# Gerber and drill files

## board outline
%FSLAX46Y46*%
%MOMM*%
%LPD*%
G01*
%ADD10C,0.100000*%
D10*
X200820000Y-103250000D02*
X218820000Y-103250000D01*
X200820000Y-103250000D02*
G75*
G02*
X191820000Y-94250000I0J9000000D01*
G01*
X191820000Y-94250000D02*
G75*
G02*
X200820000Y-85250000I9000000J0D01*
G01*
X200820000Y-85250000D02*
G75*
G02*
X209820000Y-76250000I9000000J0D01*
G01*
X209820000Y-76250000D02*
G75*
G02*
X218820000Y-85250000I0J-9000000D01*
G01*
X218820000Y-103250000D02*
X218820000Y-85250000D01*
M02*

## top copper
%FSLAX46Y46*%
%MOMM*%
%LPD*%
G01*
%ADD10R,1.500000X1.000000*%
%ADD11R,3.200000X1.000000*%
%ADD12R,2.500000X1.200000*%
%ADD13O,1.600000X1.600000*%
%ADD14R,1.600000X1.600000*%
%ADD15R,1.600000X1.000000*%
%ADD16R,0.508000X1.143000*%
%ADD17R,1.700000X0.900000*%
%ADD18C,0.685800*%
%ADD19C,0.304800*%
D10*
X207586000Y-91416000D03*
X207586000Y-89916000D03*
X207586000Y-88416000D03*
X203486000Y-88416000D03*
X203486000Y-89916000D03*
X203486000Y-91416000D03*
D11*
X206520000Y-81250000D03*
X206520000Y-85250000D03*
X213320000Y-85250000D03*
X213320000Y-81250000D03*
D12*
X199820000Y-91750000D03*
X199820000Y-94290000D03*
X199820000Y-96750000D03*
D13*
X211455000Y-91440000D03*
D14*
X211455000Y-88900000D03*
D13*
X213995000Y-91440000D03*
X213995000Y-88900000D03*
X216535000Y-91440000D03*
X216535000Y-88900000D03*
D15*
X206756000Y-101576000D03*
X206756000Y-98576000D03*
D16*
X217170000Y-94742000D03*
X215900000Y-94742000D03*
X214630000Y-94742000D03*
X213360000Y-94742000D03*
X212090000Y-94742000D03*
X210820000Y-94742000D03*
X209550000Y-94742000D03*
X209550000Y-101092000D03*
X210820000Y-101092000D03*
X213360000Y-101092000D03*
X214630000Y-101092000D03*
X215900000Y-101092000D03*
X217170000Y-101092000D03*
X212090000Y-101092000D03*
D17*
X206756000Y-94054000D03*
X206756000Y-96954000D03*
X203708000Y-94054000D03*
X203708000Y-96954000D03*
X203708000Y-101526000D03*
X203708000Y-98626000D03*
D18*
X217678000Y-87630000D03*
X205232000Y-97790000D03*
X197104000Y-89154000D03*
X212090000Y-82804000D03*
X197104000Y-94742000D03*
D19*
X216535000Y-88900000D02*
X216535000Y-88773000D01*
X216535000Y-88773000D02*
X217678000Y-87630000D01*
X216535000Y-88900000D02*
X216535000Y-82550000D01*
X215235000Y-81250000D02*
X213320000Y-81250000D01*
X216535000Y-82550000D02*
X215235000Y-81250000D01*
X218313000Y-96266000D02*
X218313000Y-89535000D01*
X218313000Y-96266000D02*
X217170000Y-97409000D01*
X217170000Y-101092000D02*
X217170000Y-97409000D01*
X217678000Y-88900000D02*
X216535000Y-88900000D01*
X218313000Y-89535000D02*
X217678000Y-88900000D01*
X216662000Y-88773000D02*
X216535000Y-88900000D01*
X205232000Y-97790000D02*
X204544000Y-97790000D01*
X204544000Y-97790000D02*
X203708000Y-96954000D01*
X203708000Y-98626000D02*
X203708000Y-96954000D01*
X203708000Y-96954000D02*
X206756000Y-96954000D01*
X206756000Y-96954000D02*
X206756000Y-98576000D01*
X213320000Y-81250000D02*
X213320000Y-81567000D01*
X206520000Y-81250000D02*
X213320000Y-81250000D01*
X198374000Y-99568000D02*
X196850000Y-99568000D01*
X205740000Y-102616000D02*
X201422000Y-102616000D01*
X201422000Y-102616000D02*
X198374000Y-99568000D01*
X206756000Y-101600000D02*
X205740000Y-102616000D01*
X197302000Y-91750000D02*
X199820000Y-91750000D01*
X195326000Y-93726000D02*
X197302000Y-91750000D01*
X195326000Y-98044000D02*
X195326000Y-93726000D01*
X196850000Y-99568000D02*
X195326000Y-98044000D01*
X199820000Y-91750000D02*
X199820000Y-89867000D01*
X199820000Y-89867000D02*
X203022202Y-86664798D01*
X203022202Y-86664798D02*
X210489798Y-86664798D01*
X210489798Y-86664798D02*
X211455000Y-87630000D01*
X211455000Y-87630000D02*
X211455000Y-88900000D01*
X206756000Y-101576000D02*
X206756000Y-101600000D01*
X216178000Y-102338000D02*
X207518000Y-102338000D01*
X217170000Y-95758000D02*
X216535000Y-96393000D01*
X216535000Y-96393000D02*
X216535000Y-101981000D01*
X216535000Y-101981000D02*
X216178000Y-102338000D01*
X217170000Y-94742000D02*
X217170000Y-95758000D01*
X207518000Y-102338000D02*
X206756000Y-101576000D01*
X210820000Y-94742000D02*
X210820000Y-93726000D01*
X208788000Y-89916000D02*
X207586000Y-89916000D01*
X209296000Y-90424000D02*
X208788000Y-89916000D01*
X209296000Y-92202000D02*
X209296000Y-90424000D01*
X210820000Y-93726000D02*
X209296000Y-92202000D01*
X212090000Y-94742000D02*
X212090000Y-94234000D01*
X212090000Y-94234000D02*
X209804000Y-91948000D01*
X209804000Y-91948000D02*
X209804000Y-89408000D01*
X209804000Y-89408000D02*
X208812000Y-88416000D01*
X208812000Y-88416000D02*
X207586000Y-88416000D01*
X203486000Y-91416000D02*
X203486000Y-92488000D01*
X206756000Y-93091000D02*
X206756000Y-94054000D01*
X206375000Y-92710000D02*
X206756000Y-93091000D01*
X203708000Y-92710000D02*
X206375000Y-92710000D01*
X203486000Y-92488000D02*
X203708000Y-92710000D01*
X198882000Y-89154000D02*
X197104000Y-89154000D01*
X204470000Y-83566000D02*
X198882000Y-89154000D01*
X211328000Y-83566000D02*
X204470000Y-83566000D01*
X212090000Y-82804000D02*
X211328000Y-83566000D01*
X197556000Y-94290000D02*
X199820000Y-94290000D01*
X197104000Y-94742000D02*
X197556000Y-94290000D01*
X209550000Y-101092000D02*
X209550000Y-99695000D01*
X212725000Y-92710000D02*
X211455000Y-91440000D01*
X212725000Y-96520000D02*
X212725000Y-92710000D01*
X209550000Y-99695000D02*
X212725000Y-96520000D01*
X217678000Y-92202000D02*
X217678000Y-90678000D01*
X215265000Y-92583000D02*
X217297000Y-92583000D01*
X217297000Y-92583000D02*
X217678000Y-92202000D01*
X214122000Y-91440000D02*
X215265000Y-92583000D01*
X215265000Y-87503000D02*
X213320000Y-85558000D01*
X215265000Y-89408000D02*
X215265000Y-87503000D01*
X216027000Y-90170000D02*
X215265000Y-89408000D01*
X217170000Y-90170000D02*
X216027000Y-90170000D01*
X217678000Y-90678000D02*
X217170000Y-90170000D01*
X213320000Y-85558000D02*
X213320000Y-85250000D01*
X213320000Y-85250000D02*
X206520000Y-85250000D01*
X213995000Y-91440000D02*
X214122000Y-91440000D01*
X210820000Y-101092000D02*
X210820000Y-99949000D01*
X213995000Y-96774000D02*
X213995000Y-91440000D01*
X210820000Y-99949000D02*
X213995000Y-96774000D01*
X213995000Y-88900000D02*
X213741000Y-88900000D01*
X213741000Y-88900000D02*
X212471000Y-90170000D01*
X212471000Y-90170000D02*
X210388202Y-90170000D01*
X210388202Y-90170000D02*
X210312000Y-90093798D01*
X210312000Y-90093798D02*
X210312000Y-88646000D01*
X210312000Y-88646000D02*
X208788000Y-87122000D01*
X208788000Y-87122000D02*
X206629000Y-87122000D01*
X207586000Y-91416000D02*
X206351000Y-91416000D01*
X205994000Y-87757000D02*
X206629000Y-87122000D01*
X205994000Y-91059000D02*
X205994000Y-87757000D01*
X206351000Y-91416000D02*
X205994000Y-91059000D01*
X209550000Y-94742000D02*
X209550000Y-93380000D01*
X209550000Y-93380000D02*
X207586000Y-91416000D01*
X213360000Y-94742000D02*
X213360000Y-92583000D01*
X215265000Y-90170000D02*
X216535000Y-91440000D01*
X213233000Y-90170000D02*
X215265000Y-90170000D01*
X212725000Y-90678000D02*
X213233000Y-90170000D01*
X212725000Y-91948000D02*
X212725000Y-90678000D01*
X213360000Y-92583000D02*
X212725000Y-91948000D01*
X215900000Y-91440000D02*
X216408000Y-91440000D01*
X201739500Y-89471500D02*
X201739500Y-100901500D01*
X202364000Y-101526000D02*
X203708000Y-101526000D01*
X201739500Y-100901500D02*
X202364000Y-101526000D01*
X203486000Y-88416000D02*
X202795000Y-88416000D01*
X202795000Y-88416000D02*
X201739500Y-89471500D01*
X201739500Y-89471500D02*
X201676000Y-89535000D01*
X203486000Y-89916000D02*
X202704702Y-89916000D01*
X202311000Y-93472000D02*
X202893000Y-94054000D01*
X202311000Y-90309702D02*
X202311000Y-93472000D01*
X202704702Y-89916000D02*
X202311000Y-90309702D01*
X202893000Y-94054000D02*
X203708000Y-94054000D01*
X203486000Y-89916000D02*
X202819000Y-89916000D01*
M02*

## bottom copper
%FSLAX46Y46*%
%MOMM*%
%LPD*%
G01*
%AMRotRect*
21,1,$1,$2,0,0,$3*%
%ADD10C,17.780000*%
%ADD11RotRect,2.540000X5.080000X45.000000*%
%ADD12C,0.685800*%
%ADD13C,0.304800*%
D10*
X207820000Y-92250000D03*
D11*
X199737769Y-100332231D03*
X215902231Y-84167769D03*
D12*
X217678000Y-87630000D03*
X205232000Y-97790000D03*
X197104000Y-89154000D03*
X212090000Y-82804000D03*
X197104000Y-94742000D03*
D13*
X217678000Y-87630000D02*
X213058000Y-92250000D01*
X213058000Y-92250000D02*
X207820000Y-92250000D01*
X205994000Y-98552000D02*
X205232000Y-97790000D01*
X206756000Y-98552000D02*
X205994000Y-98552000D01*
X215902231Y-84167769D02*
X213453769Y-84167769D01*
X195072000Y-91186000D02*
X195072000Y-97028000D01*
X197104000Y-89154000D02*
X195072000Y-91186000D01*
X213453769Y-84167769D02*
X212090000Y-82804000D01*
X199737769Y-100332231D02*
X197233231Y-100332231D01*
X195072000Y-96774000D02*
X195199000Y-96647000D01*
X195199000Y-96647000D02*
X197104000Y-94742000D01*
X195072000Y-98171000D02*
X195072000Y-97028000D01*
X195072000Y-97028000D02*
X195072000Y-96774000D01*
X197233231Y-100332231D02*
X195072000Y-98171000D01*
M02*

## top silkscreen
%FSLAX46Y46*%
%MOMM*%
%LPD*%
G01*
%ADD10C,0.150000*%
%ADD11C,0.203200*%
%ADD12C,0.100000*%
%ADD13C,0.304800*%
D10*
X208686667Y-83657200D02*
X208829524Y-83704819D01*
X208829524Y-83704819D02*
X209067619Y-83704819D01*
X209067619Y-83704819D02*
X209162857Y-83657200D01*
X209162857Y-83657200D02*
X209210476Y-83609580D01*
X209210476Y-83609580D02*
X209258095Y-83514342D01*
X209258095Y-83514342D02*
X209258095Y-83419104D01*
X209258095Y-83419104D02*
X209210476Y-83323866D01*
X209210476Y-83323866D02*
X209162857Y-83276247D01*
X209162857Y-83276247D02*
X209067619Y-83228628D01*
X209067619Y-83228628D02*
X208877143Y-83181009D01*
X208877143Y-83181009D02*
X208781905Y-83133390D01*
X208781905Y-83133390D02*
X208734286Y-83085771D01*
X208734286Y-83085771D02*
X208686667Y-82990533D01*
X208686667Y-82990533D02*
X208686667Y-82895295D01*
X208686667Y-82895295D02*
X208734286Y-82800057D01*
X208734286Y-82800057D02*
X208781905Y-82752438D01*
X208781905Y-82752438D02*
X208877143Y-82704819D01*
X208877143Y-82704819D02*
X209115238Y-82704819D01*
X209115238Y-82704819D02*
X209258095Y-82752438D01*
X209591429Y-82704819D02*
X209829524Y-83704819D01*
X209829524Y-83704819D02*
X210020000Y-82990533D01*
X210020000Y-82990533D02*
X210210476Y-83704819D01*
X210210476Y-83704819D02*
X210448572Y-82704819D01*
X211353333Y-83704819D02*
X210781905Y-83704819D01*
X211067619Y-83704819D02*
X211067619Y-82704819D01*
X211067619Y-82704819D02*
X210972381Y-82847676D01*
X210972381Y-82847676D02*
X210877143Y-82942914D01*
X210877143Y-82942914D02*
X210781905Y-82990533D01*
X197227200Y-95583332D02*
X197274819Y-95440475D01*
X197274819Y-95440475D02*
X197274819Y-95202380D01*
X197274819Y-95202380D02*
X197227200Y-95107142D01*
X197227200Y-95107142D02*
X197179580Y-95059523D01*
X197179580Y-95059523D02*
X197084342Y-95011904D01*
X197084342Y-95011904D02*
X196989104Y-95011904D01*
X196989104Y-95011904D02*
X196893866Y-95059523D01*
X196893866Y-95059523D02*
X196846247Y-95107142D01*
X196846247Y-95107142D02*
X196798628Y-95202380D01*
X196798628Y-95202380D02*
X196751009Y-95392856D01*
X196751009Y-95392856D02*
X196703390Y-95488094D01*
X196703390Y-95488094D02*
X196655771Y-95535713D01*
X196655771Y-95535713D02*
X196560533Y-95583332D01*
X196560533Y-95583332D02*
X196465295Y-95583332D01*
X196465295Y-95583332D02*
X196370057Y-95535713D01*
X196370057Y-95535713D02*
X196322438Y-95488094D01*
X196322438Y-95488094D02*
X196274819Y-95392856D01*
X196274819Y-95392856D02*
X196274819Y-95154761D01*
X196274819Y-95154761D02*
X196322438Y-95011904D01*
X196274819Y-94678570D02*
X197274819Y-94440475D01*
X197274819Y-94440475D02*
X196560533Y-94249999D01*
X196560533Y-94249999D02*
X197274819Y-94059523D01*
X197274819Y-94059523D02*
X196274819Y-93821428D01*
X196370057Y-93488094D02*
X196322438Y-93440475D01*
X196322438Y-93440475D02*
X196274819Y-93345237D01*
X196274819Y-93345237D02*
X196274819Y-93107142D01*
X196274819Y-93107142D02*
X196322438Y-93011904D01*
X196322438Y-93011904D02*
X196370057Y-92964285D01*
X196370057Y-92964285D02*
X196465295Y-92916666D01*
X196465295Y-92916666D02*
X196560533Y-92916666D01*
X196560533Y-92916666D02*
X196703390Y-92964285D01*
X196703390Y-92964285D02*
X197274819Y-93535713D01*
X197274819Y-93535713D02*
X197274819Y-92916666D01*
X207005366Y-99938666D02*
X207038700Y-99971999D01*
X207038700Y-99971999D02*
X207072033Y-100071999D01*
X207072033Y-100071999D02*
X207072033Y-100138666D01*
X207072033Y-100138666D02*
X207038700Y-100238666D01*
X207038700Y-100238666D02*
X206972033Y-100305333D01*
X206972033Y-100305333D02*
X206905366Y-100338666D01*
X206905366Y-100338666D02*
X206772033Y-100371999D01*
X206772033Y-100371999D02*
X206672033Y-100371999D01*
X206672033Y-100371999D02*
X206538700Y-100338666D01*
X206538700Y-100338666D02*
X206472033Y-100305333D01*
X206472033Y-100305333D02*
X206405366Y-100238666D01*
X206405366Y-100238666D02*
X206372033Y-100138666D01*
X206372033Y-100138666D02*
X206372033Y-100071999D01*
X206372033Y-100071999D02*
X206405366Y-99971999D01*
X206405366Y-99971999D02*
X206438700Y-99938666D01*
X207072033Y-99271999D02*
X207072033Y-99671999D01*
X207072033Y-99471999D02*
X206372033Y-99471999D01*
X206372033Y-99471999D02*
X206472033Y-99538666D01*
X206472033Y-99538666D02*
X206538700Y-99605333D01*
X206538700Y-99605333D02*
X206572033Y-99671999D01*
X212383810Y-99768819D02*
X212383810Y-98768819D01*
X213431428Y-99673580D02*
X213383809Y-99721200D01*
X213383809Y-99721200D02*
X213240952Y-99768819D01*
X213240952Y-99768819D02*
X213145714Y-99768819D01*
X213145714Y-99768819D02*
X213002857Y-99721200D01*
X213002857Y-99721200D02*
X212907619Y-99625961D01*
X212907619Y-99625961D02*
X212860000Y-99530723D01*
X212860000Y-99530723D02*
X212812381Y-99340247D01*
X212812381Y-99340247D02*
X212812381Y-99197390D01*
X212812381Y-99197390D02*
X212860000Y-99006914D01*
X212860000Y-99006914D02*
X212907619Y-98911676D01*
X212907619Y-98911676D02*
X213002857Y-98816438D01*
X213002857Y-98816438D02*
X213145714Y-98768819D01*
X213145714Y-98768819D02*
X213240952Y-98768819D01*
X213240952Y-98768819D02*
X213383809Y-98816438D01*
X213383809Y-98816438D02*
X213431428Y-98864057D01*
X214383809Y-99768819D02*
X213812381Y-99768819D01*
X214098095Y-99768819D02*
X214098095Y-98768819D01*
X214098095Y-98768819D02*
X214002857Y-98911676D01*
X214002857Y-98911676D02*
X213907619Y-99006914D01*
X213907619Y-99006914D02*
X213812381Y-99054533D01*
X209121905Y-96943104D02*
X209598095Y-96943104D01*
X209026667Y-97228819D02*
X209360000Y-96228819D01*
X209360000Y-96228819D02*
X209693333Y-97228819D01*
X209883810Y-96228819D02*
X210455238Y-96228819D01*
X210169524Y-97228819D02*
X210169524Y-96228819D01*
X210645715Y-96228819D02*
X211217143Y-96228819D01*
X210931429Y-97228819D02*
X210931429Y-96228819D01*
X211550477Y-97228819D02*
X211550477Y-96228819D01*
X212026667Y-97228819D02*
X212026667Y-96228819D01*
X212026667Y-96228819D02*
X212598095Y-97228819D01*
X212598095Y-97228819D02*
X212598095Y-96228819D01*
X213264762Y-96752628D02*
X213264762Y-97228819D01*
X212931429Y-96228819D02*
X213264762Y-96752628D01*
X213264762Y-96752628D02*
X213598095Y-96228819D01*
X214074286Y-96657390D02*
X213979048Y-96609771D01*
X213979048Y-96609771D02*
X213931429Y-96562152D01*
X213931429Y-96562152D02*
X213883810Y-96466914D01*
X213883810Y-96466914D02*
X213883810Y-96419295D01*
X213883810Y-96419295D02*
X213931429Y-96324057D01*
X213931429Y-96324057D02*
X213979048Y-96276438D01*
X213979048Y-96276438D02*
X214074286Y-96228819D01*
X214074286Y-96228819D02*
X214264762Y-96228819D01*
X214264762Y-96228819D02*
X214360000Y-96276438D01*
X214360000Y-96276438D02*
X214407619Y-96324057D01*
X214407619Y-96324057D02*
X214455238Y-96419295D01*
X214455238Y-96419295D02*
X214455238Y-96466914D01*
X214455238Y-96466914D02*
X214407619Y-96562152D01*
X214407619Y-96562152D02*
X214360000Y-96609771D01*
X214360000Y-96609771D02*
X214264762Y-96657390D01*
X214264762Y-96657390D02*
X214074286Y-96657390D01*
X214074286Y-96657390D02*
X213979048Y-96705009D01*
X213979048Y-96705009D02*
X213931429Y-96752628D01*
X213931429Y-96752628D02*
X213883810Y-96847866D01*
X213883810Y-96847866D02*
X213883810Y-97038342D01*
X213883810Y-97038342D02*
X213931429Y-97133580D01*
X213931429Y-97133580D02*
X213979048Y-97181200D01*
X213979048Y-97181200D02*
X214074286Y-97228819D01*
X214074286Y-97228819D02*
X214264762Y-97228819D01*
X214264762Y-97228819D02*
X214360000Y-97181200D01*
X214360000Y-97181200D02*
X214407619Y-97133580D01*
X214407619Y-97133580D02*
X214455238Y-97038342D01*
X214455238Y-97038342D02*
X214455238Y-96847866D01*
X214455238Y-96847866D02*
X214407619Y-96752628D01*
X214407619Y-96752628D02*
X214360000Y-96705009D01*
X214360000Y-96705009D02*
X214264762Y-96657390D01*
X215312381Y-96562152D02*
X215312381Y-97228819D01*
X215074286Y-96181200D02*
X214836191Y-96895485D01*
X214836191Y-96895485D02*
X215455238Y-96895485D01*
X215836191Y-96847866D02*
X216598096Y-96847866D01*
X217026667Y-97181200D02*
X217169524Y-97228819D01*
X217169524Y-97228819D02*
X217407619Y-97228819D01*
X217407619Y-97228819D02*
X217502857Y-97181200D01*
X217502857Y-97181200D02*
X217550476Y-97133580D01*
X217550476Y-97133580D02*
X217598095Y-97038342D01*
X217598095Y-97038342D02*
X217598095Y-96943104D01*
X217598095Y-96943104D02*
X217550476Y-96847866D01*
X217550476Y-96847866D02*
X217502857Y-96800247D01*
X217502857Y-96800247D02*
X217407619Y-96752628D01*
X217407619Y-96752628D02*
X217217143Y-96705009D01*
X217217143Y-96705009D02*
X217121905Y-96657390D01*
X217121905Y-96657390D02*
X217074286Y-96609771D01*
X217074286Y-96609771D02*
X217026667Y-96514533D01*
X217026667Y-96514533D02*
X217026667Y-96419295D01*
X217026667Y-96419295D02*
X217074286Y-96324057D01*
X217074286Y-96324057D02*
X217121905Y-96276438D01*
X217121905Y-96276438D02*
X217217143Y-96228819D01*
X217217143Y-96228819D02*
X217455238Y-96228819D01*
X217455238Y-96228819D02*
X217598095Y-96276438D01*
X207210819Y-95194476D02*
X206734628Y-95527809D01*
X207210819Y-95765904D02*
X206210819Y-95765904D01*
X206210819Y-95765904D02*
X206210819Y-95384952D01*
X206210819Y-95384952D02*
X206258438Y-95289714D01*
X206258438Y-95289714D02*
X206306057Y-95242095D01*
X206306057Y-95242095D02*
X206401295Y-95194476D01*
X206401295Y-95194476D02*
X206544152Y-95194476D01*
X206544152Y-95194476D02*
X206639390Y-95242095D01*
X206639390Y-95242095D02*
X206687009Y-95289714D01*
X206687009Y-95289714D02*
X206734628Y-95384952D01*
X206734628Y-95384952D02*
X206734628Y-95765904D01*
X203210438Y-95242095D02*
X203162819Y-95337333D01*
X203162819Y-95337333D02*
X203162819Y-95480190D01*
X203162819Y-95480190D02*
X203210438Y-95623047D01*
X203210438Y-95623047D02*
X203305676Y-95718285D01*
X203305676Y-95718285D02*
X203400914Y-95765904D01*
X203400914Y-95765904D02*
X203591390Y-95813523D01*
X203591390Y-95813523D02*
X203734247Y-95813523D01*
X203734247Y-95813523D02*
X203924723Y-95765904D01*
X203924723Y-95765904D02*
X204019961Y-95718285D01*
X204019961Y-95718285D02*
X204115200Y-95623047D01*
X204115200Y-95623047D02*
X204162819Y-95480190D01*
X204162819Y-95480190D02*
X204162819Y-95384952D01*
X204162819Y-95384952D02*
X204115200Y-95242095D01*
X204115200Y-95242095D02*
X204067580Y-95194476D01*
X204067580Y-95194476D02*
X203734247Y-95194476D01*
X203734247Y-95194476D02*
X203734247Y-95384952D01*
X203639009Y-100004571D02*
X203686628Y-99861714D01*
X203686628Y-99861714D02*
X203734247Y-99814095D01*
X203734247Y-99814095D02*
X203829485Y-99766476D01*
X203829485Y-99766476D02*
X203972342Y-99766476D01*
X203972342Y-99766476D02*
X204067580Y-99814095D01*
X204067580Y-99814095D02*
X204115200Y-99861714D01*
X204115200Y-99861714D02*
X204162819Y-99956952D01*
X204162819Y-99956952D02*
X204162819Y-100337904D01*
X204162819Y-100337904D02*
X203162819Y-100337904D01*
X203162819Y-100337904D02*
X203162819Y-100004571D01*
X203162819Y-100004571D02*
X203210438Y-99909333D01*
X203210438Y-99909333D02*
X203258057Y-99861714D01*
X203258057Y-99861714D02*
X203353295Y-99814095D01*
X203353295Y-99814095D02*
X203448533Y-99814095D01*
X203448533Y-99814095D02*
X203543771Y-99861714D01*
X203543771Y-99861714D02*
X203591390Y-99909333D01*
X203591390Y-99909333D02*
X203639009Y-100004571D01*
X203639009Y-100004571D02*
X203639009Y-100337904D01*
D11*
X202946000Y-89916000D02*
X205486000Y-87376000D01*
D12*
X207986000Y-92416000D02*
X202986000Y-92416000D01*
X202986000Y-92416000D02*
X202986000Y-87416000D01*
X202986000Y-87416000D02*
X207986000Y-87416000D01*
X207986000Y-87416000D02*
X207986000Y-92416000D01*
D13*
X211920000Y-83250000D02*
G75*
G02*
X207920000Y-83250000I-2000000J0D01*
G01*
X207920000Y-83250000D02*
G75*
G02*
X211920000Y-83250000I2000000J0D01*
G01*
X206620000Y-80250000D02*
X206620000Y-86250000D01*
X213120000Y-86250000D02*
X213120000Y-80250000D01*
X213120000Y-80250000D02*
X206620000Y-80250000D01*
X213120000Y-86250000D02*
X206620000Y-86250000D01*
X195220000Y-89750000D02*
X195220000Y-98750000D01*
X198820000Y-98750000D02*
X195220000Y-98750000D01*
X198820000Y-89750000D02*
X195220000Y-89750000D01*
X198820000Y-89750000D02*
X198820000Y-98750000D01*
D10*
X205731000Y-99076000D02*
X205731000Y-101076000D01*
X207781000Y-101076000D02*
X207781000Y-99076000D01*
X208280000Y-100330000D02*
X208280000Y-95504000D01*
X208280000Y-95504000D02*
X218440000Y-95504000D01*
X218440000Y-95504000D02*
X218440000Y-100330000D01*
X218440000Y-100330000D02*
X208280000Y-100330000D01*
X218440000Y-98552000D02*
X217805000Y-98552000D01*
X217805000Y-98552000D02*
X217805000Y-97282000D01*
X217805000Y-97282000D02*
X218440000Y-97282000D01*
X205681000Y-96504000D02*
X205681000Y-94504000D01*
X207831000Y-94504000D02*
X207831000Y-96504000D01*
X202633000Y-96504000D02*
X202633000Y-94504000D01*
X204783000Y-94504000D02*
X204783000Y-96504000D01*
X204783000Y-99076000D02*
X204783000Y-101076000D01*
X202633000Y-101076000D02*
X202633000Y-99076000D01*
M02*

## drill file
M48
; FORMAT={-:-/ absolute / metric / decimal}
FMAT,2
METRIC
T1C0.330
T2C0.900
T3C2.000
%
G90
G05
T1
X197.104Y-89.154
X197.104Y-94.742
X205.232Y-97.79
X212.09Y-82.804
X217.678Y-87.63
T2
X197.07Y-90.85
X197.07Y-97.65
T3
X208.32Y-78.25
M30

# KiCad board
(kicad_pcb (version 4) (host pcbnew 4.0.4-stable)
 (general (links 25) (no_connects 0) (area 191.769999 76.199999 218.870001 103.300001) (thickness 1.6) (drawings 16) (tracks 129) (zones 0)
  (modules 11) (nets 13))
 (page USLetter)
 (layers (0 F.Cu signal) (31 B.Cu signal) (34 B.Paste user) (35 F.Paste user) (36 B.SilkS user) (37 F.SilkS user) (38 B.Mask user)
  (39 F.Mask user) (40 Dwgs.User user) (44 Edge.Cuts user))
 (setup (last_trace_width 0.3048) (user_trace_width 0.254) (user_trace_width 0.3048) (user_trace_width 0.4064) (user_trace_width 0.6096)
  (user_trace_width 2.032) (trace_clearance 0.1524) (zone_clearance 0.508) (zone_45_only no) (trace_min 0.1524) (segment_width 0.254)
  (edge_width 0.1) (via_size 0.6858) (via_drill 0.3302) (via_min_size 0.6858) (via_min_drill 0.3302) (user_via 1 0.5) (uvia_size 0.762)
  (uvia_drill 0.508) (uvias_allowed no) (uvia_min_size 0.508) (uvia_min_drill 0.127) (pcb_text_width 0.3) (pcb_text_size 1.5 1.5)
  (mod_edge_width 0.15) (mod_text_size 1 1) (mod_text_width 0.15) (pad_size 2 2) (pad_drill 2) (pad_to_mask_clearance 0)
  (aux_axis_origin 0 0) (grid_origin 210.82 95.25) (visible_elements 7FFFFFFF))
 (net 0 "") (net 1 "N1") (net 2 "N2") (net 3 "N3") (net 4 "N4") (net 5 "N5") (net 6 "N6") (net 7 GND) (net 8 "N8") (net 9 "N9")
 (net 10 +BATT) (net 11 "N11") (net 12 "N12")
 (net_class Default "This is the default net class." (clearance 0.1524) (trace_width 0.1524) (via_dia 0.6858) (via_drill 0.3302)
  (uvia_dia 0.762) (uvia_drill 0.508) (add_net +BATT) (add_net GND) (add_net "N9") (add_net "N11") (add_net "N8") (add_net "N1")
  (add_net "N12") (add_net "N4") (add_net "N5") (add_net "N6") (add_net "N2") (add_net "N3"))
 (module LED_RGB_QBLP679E (layer F.Cu) (at 205.486 89.916 180)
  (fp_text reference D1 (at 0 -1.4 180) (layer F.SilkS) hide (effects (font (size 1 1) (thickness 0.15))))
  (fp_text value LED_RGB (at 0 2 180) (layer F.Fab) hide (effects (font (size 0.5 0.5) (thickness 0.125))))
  (fp_line (start 2.54 0) (end 0 2.54) (layer F.SilkS) (width 0.2032))
  (fp_line (start -2.5 -2.5) (end 2.5 -2.5) (layer F.SilkS) (width 0.1))
  (fp_line (start 2.5 -2.5) (end 2.5 2.5) (layer F.SilkS) (width 0.1))
  (fp_line (start 2.5 2.5) (end -2.5 2.5) (layer F.SilkS) (width 0.1))
  (fp_line (start -2.5 2.5) (end -2.5 -2.5) (layer F.SilkS) (width 0.1))
  (pad 4 smd rect (at -2.1 -1.5 270) (size 1 1.5) (layers F.Cu F.Paste F.Mask) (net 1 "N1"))
  (pad 5 smd rect (at -2.1 0 270) (size 1 1.5) (layers F.Cu F.Paste F.Mask) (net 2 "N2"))
  (pad 6 smd rect (at -2.1 1.5 270) (size 1 1.5) (layers F.Cu F.Paste F.Mask) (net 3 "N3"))
  (pad 1 smd rect (at 2 1.5 270) (size 1 1.5) (layers F.Cu F.Paste F.Mask) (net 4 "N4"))
  (pad 2 smd rect (at 2 0 270) (size 1 1.5) (layers F.Cu F.Paste F.Mask) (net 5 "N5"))
  (pad 3 smd rect (at 2 -1.5 270) (size 1 1.5) (layers F.Cu F.Paste F.Mask) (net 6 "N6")))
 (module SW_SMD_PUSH (layer F.Cu) (at 213.32 85.25 180)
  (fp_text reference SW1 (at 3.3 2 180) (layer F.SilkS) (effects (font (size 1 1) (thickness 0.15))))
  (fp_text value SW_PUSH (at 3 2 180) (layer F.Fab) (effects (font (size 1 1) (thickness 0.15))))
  (fp_circle (center 3.4 2) (end 3.4 0) (layer F.SilkS) (width 0.3048))
  (fp_line (start 6.7 5) (end 6.7 -1) (layer F.SilkS) (width 0.3048))
  (fp_line (start 0.2 -1) (end 0.2 5) (layer F.SilkS) (width 0.3048))
  (fp_line (start 0.2 5) (end 6.7 5) (layer F.SilkS) (width 0.3048))
  (fp_line (start 0.2 -1) (end 6.7 -1) (layer F.SilkS) (width 0.3048))
  (pad 2 smd rect (at 6.8 4 180) (size 3.2 1) (layers F.Cu F.Paste F.Mask) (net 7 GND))
  (pad 1 smd rect (at 6.8 0 180) (size 3.2 1) (layers F.Cu F.Paste F.Mask) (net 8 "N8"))
  (pad 1 smd rect (at 0 0 180) (size 3.2 1) (layers F.Cu F.Paste F.Mask) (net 8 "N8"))
  (pad 2 smd rect (at 0 4 180) (size 3.2 1) (layers F.Cu F.Paste F.Mask) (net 7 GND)))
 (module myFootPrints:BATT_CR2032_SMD (layer B.Cu) (at 207.82 92.25 45)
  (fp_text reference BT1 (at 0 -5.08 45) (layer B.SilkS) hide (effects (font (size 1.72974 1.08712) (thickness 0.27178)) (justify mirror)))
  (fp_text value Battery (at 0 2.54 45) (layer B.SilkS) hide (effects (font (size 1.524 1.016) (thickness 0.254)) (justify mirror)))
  (pad 2 smd circle (at 0 0 45) (size 17.78 17.78) (layers B.Cu B.Paste B.Mask) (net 7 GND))
  (pad 1 smd rect (at -11.43 0 45) (size 2.54 5.08) (layers B.Cu B.Paste B.Mask) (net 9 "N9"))
  (pad 1 smd rect (at 11.43 0 45) (size 2.54 5.08) (layers B.Cu B.Paste B.Mask) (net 9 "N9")))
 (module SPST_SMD (layer F.Cu) (at 199.82 94.25 270)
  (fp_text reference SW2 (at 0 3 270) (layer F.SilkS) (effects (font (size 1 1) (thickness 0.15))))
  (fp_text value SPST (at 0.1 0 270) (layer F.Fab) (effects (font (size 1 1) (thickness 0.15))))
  (fp_line (start -4.5 4.6) (end 4.5 4.6) (layer F.SilkS) (width 0.3048))
  (fp_line (start 4.5 1) (end 4.5 4.6) (layer F.SilkS) (width 0.3048))
  (fp_line (start -4.5 1) (end -4.5 4.6) (layer F.SilkS) (width 0.3048))
  (fp_line (start -4.5 1) (end 4.5 1) (layer F.SilkS) (width 0.3048))
  (pad "" np_thru_hole circle (at 3.4 2.75 270) (size 0.9 0.9) (drill 0.9) (layers *.Cu *.Mask))
  (pad 1 smd rect (at -2.5 0 270) (size 1.2 2.5) (layers F.Cu F.Paste F.Mask) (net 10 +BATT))
  (pad 2 smd rect (at 0.04 0 270) (size 1.2 2.5) (layers F.Cu F.Paste F.Mask) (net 9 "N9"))
  (pad 3 smd rect (at 2.5 0 270) (size 1.2 2.5) (layers F.Cu F.Paste F.Mask))
  (pad "" np_thru_hole circle (at -3.4 2.75 270) (size 0.9 0.9) (drill 0.9) (layers *.Cu *.Mask)))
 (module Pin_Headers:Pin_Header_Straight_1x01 (layer F.Cu) (at 208.32 78.25)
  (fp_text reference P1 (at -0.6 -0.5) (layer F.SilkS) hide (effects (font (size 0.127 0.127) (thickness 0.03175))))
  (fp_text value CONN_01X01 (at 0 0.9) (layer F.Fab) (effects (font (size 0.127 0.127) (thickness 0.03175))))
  (pad "" np_thru_hole circle (at 0 0) (size 2 2) (drill 2) (layers *.Cu *.Mask)))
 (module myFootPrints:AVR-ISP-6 (layer F.Cu) (at 211.455 91.44 90)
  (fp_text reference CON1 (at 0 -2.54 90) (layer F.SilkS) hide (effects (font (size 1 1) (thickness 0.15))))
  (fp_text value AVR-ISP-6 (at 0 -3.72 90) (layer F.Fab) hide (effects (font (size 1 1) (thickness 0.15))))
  (pad 1 smd oval (at 0 0 90) (size 1.6 1.6) (layers F.Cu F.Paste F.Mask) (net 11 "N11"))
  (pad 2 smd rect (at 2.54 0 90) (size 1.6 1.6) (layers F.Cu F.Paste F.Mask) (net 10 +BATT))
  (pad 3 smd oval (at 0 2.54 90) (size 1.6 1.6) (layers F.Cu F.Paste F.Mask) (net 8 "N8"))
  (pad 4 smd oval (at 2.54 2.54 90) (size 1.6 1.6) (layers F.Cu F.Paste F.Mask) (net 1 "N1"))
  (pad 5 smd oval (at 0 5.08 90) (size 1.6 1.6) (layers F.Cu F.Paste F.Mask) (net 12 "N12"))
  (pad 6 smd oval (at 2.54 5.08 90) (size 1.6 1.6) (layers F.Cu F.Paste F.Mask) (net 7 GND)))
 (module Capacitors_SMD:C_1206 (layer F.Cu) (at 206.756 100.076 90)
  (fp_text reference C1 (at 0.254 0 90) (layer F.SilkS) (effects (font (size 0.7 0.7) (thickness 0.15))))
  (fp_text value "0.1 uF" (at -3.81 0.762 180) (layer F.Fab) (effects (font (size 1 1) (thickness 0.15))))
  (fp_line (start 1 -1.025) (end -1 -1.025) (layer F.SilkS) (width 0.15))
  (fp_line (start -1 1.025) (end 1 1.025) (layer F.SilkS) (width 0.15))
  (pad 1 smd rect (at -1.5 0 90) (size 1 1.6) (layers F.Cu F.Paste F.Mask) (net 10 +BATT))
  (pad 2 smd rect (at 1.5 0 90) (size 1 1.6) (layers F.Cu F.Paste F.Mask) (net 7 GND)))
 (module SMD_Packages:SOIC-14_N (layer F.Cu) (at 213.36 98.044 180)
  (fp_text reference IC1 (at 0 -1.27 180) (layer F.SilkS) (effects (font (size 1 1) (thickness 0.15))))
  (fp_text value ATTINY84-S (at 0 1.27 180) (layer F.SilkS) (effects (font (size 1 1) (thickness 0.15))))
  (fp_line (start 5.08 -2.286) (end 5.08 2.54) (layer F.SilkS) (width 0.15))
  (fp_line (start 5.08 2.54) (end -5.08 2.54) (layer F.SilkS) (width 0.15))
  (fp_line (start -5.08 2.54) (end -5.08 -2.286) (layer F.SilkS) (width 0.15))
  (fp_line (start -5.08 -2.286) (end 5.08 -2.286) (layer F.SilkS) (width 0.15))
  (fp_line (start -5.08 -0.508) (end -4.445 -0.508) (layer F.SilkS) (width 0.15))
  (fp_line (start -4.445 -0.508) (end -4.445 0.762) (layer F.SilkS) (width 0.15))
  (fp_line (start -4.445 0.762) (end -5.08 0.762) (layer F.SilkS) (width 0.15))
  (pad 1 smd rect (at -3.81 3.302 180) (size 0.508 1.143) (layers F.Cu F.Paste F.Mask) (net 10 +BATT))
  (pad 2 smd rect (at -2.54 3.302 180) (size 0.508 1.143) (layers F.Cu F.Paste F.Mask))
  (pad 3 smd rect (at -1.27 3.302 180) (size 0.508 1.143) (layers F.Cu F.Paste F.Mask))
  (pad 4 smd rect (at 0 3.302 180) (size 0.508 1.143) (layers F.Cu F.Paste F.Mask) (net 12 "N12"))
  (pad 5 smd rect (at 1.27 3.302 180) (size 0.508 1.143) (layers F.Cu F.Paste F.Mask) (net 3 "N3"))
  (pad 6 smd rect (at 2.54 3.302 180) (size 0.508 1.143) (layers F.Cu F.Paste F.Mask) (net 2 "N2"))
  (pad 7 smd rect (at 3.81 3.302 180) (size 0.508 1.143) (layers F.Cu F.Paste F.Mask) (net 1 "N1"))
  (pad 8 smd rect (at 3.81 -3.048 180) (size 0.508 1.143) (layers F.Cu F.Paste F.Mask) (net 11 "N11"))
  (pad 9 smd rect (at 2.54 -3.048 180) (size 0.508 1.143) (layers F.Cu F.Paste F.Mask) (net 8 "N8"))
  (pad 11 smd rect (at 0 -3.048 180) (size 0.508 1.143) (layers F.Cu F.Paste F.Mask))
  (pad 12 smd rect (at -1.27 -3.048 180) (size 0.508 1.143) (layers F.Cu F.Paste F.Mask))
  (pad 13 smd rect (at -2.54 -3.048 180) (size 0.508 1.143) (layers F.Cu F.Paste F.Mask))
  (pad 14 smd rect (at -3.81 -3.048 180) (size 0.508 1.143) (layers F.Cu F.Paste F.Mask) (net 7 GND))
  (pad 10 smd rect (at 1.27 -3.048 180) (size 0.508 1.143) (layers F.Cu F.Paste F.Mask)))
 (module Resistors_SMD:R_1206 (layer F.Cu) (at 206.756 95.504 270)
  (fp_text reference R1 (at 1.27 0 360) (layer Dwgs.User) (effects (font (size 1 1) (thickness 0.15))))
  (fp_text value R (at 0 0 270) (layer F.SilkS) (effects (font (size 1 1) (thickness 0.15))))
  (fp_line (start 1 1.075) (end -1 1.075) (layer F.SilkS) (width 0.15))
  (fp_line (start -1 -1.075) (end 1 -1.075) (layer F.SilkS) (width 0.15))
  (pad 1 smd rect (at -1.45 0 270) (size 0.9 1.7) (layers F.Cu F.Paste F.Mask) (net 6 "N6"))
  (pad 2 smd rect (at 1.45 0 270) (size 0.9 1.7) (layers F.Cu F.Paste F.Mask) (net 7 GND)))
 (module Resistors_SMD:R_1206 (layer F.Cu) (at 203.708 95.504 270)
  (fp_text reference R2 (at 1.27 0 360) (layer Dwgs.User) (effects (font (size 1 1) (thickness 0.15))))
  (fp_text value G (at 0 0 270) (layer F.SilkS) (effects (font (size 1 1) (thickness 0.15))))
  (fp_line (start 1 1.075) (end -1 1.075) (layer F.SilkS) (width 0.15))
  (fp_line (start -1 -1.075) (end 1 -1.075) (layer F.SilkS) (width 0.15))
  (pad 1 smd rect (at -1.45 0 270) (size 0.9 1.7) (layers F.Cu F.Paste F.Mask) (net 5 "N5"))
  (pad 2 smd rect (at 1.45 0 270) (size 0.9 1.7) (layers F.Cu F.Paste F.Mask) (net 7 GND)))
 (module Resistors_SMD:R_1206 (layer F.Cu) (at 203.708 100.076 90)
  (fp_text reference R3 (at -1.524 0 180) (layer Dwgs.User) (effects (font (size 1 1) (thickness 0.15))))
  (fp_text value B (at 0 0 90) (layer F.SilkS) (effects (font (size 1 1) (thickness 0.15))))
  (fp_line (start 1 1.075) (end -1 1.075) (layer F.SilkS) (width 0.15))
  (fp_line (start -1 -1.075) (end 1 -1.075) (layer F.SilkS) (width 0.15))
  (pad 1 smd rect (at -1.45 0 90) (size 0.9 1.7) (layers F.Cu F.Paste F.Mask) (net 4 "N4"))
  (pad 2 smd rect (at 1.45 0 90) (size 0.9 1.7) (layers F.Cu F.Paste F.Mask) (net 7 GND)))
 (gr_line (start 200.82 103.25) (end 218.82 103.25) (angle 90) (layer Edge.Cuts) (width 0.1))
 (gr_arc (start 200.82 94.25) (end 200.82 103.25) (angle 90) (layer Edge.Cuts) (width 0.1))
 (gr_arc (start 200.82 94.25) (end 191.82 94.25) (angle 90) (layer Edge.Cuts) (width 0.1))
 (gr_arc (start 209.82 85.25) (end 200.82 85.25) (angle 90) (layer Edge.Cuts) (width 0.1))
 (gr_arc (start 209.82 85.25) (end 209.82 76.25) (angle 90) (layer Edge.Cuts) (width 0.1))
 (gr_line (start 218.82 103.25) (end 218.82 85.25) (angle 90) (layer Edge.Cuts) (width 0.1))
 (segment (start 216.535 88.9) (end 216.535 88.773) (width 0.3048) (layer F.Cu) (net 7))
 (segment (start 216.535 88.773) (end 217.678 87.63) (width 0.3048) (layer F.Cu) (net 7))
 (segment (start 217.678 87.63) (end 213.058 92.25) (width 0.3048) (layer B.Cu) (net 7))
 (via (at 217.678 87.63) (size 0.6858) (drill 0.3302) (layers F.Cu B.Cu) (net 7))
 (segment (start 213.058 92.25) (end 207.82 92.25) (width 0.3048) (layer B.Cu) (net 7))
 (segment (start 216.535 88.9) (end 216.535 82.55) (width 0.3048) (layer F.Cu) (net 7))
 (segment (start 215.235 81.25) (end 213.32 81.25) (width 0.3048) (layer F.Cu) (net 7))
 (segment (start 216.535 82.55) (end 215.235 81.25) (width 0.3048) (layer F.Cu) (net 7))
 (segment (start 218.313 96.266) (end 218.313 89.535) (width 0.3048) (layer F.Cu) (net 7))
 (segment (start 218.313 96.266) (end 217.17 97.409) (width 0.3048) (layer F.Cu) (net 7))
 (segment (start 217.17 101.092) (end 217.17 97.409) (width 0.3048) (layer F.Cu) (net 7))
 (segment (start 217.678 88.9) (end 216.535 88.9) (width 0.3048) (layer F.Cu) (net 7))
 (segment (start 218.313 89.535) (end 217.678 88.9) (width 0.3048) (layer F.Cu) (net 7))
 (segment (start 216.662 88.773) (end 216.535 88.9) (width 0.3048) (layer F.Cu) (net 7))
 (segment (start 205.232 97.79) (end 204.544 97.79) (width 0.3048) (layer F.Cu) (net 7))
 (segment (start 205.994 98.552) (end 205.232 97.79) (width 0.3048) (layer B.Cu) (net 7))
 (via (at 205.232 97.79) (size 0.6858) (drill 0.3302) (layers F.Cu B.Cu) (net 7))
 (segment (start 204.544 97.79) (end 203.708 96.954) (width 0.3048) (layer F.Cu) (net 7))
 (segment (start 206.756 98.552) (end 205.994 98.552) (width 0.3048) (layer B.Cu) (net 7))
 (segment (start 203.708 98.626) (end 203.708 96.954) (width 0.3048) (layer F.Cu) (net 7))
 (segment (start 203.708 96.954) (end 206.756 96.954) (width 0.3048) (layer F.Cu) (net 7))
 (segment (start 206.756 96.954) (end 206.756 98.576) (width 0.3048) (layer F.Cu) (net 7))
 (segment (start 213.32 81.25) (end 213.32 81.567) (width 0.3048) (layer F.Cu) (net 7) (status 30))
 (segment (start 206.52 81.25) (end 213.32 81.25) (width 0.3048) (layer F.Cu) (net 7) (status 30))
 (segment (start 198.374 99.568) (end 196.85 99.568) (width 0.3048) (layer F.Cu) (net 10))
 (segment (start 205.74 102.616) (end 201.422 102.616) (width 0.3048) (layer F.Cu) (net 10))
 (segment (start 201.422 102.616) (end 198.374 99.568) (width 0.3048) (layer F.Cu) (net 10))
 (segment (start 206.756 101.6) (end 205.74 102.616) (width 0.3048) (layer F.Cu) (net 10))
 (segment (start 197.302 91.75) (end 199.82 91.75) (width 0.3048) (layer F.Cu) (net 10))
 (segment (start 195.326 93.726) (end 197.302 91.75) (width 0.3048) (layer F.Cu) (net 10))
 (segment (start 195.326 98.044) (end 195.326 93.726) (width 0.3048) (layer F.Cu) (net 10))
 (segment (start 196.85 99.568) (end 195.326 98.044) (width 0.3048) (layer F.Cu) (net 10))
 (segment (start 199.82 91.75) (end 199.82 89.867) (width 0.3048) (layer F.Cu) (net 10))
 (segment (start 199.82 89.867) (end 203.022202 86.664798) (width 0.3048) (layer F.Cu) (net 10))
 (segment (start 203.022202 86.664798) (end 210.489798 86.664798) (width 0.3048) (layer F.Cu) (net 10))
 (segment (start 210.489798 86.664798) (end 211.455 87.63) (width 0.3048) (layer F.Cu) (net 10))
 (segment (start 211.455 87.63) (end 211.455 88.9) (width 0.3048) (layer F.Cu) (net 10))
 (segment (start 206.756 101.576) (end 206.756 101.6) (width 0.3048) (layer F.Cu) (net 10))
 (segment (start 216.178 102.338) (end 207.518 102.338) (width 0.3048) (layer F.Cu) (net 10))
 (segment (start 217.17 95.758) (end 216.535 96.393) (width 0.3048) (layer F.Cu) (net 10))
 (segment (start 216.535 96.393) (end 216.535 101.981) (width 0.3048) (layer F.Cu) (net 10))
 (segment (start 216.535 101.981) (end 216.178 102.338) (width 0.3048) (layer F.Cu) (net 10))
 (segment (start 217.17 94.742) (end 217.17 95.758) (width 0.3048) (layer F.Cu) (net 10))
 (segment (start 207.518 102.338) (end 206.756 101.576) (width 0.3048) (layer F.Cu) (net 10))
 (segment (start 210.82 94.742) (end 210.82 93.726) (width 0.3048) (layer F.Cu) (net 2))
 (segment (start 208.788 89.916) (end 207.586 89.916) (width 0.3048) (layer F.Cu) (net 2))
 (segment (start 209.296 90.424) (end 208.788 89.916) (width 0.3048) (layer F.Cu) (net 2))
 (segment (start 209.296 92.202) (end 209.296 90.424) (width 0.3048) (layer F.Cu) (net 2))
 (segment (start 210.82 93.726) (end 209.296 92.202) (width 0.3048) (layer F.Cu) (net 2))
 (segment (start 212.09 94.742) (end 212.09 94.234) (width 0.3048) (layer F.Cu) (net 3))
 (segment (start 212.09 94.234) (end 209.804 91.948) (width 0.3048) (layer F.Cu) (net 3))
 (segment (start 209.804 91.948) (end 209.804 89.408) (width 0.3048) (layer F.Cu) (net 3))
 (segment (start 209.804 89.408) (end 208.812 88.416) (width 0.3048) (layer F.Cu) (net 3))
 (segment (start 208.812 88.416) (end 207.586 88.416) (width 0.3048) (layer F.Cu) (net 3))
 (segment (start 203.486 91.416) (end 203.486 92.488) (width 0.3048) (layer F.Cu) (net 6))
 (segment (start 206.756 93.091) (end 206.756 94.054) (width 0.3048) (layer F.Cu) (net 6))
 (segment (start 206.375 92.71) (end 206.756 93.091) (width 0.3048) (layer F.Cu) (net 6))
 (segment (start 203.708 92.71) (end 206.375 92.71) (width 0.3048) (layer F.Cu) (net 6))
 (segment (start 203.486 92.488) (end 203.708 92.71) (width 0.3048) (layer F.Cu) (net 6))
 (segment (start 215.902231 84.167769) (end 213.453769 84.167769) (width 0.3048) (layer B.Cu) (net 9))
 (segment (start 195.072 91.186) (end 195.072 97.028) (width 0.3048) (layer B.Cu) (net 9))
 (segment (start 197.104 89.154) (end 195.072 91.186) (width 0.3048) (layer B.Cu) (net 9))
 (via (at 197.104 89.154) (size 0.6858) (drill 0.3302) (layers F.Cu B.Cu) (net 9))
 (segment (start 198.882 89.154) (end 197.104 89.154) (width 0.3048) (layer F.Cu) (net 9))
 (segment (start 204.47 83.566) (end 198.882 89.154) (width 0.3048) (layer F.Cu) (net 9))
 (segment (start 211.328 83.566) (end 204.47 83.566) (width 0.3048) (layer F.Cu) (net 9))
 (segment (start 212.09 82.804) (end 211.328 83.566) (width 0.3048) (layer F.Cu) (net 9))
 (via (at 212.09 82.804) (size 0.6858) (drill 0.3302) (layers F.Cu B.Cu) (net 9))
 (segment (start 213.453769 84.167769) (end 212.09 82.804) (width 0.3048) (layer B.Cu) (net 9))
 (segment (start 199.737769 100.332231) (end 197.233231 100.332231) (width 0.3048) (layer B.Cu) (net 9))
 (segment (start 197.556 94.29) (end 199.82 94.29) (width 0.3048) (layer F.Cu) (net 9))
 (segment (start 197.104 94.742) (end 197.556 94.29) (width 0.3048) (layer F.Cu) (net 9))
 (via (at 197.104 94.742) (size 0.6858) (drill 0.3302) (layers F.Cu B.Cu) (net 9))
 (segment (start 195.072 96.774) (end 195.199 96.647) (width 0.3048) (layer B.Cu) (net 9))
 (segment (start 195.199 96.647) (end 197.104 94.742) (width 0.3048) (layer B.Cu) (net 9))
 (segment (start 195.072 98.171) (end 195.072 97.028) (width 0.3048) (layer B.Cu) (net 9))
 (segment (start 195.072 97.028) (end 195.072 96.774) (width 0.3048) (layer B.Cu) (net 9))
 (segment (start 197.233231 100.332231) (end 195.072 98.171) (width 0.3048) (layer B.Cu) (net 9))
 (segment (start 209.55 101.092) (end 209.55 99.695) (width 0.3048) (layer F.Cu) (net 11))
 (segment (start 212.725 92.71) (end 211.455 91.44) (width 0.3048) (layer F.Cu) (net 11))
 (segment (start 212.725 96.52) (end 212.725 92.71) (width 0.3048) (layer F.Cu) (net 11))
 (segment (start 209.55 99.695) (end 212.725 96.52) (width 0.3048) (layer F.Cu) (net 11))
 (segment (start 217.678 92.202) (end 217.678 90.678) (width 0.3048) (layer F.Cu) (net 8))
 (segment (start 215.265 92.583) (end 217.297 92.583) (width 0.3048) (layer F.Cu) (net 8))
 (segment (start 217.297 92.583) (end 217.678 92.202) (width 0.3048) (layer F.Cu) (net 8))
 (segment (start 214.122 91.44) (end 215.265 92.583) (width 0.3048) (layer F.Cu) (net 8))
 (segment (start 215.265 87.503) (end 213.32 85.558) (width 0.3048) (layer F.Cu) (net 8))
 (segment (start 215.265 89.408) (end 215.265 87.503) (width 0.3048) (layer F.Cu) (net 8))
 (segment (start 216.027 90.17) (end 215.265 89.408) (width 0.3048) (layer F.Cu) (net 8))
 (segment (start 217.17 90.17) (end 216.027 90.17) (width 0.3048) (layer F.Cu) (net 8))
 (segment (start 217.678 90.678) (end 217.17 90.17) (width 0.3048) (layer F.Cu) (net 8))
 (segment (start 213.32 85.558) (end 213.32 85.25) (width 0.3048) (layer F.Cu) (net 8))
 (segment (start 213.32 85.25) (end 206.52 85.25) (width 0.3048) (layer F.Cu) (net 8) (status 30))
 (segment (start 213.995 91.44) (end 214.122 91.44) (width 0.3048) (layer F.Cu) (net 8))
 (segment (start 210.82 101.092) (end 210.82 99.949) (width 0.3048) (layer F.Cu) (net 8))
 (segment (start 213.995 96.774) (end 213.995 91.44) (width 0.3048) (layer F.Cu) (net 8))
 (segment (start 210.82 99.949) (end 213.995 96.774) (width 0.3048) (layer F.Cu) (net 8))
 (segment (start 213.995 88.9) (end 213.741 88.9) (width 0.3048) (layer F.Cu) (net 1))
 (segment (start 213.741 88.9) (end 212.471 90.17) (width 0.3048) (layer F.Cu) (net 1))
 (segment (start 212.471 90.17) (end 210.388202 90.17) (width 0.3048) (layer F.Cu) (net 1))
 (segment (start 210.388202 90.17) (end 210.312 90.093798) (width 0.3048) (layer F.Cu) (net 1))
 (segment (start 210.312 90.093798) (end 210.312 88.646) (width 0.3048) (layer F.Cu) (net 1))
 (segment (start 210.312 88.646) (end 208.788 87.122) (width 0.3048) (layer F.Cu) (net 1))
 (segment (start 208.788 87.122) (end 206.629 87.122) (width 0.3048) (layer F.Cu) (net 1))
 (segment (start 207.586 91.416) (end 206.351 91.416) (width 0.3048) (layer F.Cu) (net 1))
 (segment (start 205.994 87.757) (end 206.629 87.122) (width 0.3048) (layer F.Cu) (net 1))
 (segment (start 205.994 91.059) (end 205.994 87.757) (width 0.3048) (layer F.Cu) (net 1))
 (segment (start 206.351 91.416) (end 205.994 91.059) (width 0.3048) (layer F.Cu) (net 1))
 (segment (start 209.55 94.742) (end 209.55 93.38) (width 0.3048) (layer F.Cu) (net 1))
 (segment (start 209.55 93.38) (end 207.586 91.416) (width 0.3048) (layer F.Cu) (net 1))
 (segment (start 213.36 94.742) (end 213.36 92.583) (width 0.3048) (layer F.Cu) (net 12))
 (segment (start 215.265 90.17) (end 216.535 91.44) (width 0.3048) (layer F.Cu) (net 12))
 (segment (start 213.233 90.17) (end 215.265 90.17) (width 0.3048) (layer F.Cu) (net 12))
 (segment (start 212.725 90.678) (end 213.233 90.17) (width 0.3048) (layer F.Cu) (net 12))
 (segment (start 212.725 91.948) (end 212.725 90.678) (width 0.3048) (layer F.Cu) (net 12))
 (segment (start 213.36 92.583) (end 212.725 91.948) (width 0.3048) (layer F.Cu) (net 12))
 (segment (start 215.9 91.44) (end 216.408 91.44) (width 0.3048) (layer F.Cu) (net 12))
 (segment (start 201.7395 89.4715) (end 201.7395 100.9015) (width 0.3048) (layer F.Cu) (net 4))
 (segment (start 202.364 101.526) (end 203.708 101.526) (width 0.3048) (layer F.Cu) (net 4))
 (segment (start 201.7395 100.9015) (end 202.364 101.526) (width 0.3048) (layer F.Cu) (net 4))
 (segment (start 203.486 88.416) (end 202.795 88.416) (width 0.3048) (layer F.Cu) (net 4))
 (segment (start 202.795 88.416) (end 201.7395 89.4715) (width 0.3048) (layer F.Cu) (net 4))
 (segment (start 201.7395 89.4715) (end 201.676 89.535) (width 0.3048) (layer F.Cu) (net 4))
 (segment (start 203.486 89.916) (end 202.704702 89.916) (width 0.3048) (layer F.Cu) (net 5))
 (segment (start 202.311 93.472) (end 202.893 94.054) (width 0.3048) (layer F.Cu) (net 5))
 (segment (start 202.311 90.309702) (end 202.311 93.472) (width 0.3048) (layer F.Cu) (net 5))
 (segment (start 202.704702 89.916) (end 202.311 90.309702) (width 0.3048) (layer F.Cu) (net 5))
 (segment (start 202.893 94.054) (end 203.708 94.054) (width 0.3048) (layer F.Cu) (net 5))
 (segment (start 203.486 89.916) (end 202.819 89.916) (width 0.3048) (layer F.Cu) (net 5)))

